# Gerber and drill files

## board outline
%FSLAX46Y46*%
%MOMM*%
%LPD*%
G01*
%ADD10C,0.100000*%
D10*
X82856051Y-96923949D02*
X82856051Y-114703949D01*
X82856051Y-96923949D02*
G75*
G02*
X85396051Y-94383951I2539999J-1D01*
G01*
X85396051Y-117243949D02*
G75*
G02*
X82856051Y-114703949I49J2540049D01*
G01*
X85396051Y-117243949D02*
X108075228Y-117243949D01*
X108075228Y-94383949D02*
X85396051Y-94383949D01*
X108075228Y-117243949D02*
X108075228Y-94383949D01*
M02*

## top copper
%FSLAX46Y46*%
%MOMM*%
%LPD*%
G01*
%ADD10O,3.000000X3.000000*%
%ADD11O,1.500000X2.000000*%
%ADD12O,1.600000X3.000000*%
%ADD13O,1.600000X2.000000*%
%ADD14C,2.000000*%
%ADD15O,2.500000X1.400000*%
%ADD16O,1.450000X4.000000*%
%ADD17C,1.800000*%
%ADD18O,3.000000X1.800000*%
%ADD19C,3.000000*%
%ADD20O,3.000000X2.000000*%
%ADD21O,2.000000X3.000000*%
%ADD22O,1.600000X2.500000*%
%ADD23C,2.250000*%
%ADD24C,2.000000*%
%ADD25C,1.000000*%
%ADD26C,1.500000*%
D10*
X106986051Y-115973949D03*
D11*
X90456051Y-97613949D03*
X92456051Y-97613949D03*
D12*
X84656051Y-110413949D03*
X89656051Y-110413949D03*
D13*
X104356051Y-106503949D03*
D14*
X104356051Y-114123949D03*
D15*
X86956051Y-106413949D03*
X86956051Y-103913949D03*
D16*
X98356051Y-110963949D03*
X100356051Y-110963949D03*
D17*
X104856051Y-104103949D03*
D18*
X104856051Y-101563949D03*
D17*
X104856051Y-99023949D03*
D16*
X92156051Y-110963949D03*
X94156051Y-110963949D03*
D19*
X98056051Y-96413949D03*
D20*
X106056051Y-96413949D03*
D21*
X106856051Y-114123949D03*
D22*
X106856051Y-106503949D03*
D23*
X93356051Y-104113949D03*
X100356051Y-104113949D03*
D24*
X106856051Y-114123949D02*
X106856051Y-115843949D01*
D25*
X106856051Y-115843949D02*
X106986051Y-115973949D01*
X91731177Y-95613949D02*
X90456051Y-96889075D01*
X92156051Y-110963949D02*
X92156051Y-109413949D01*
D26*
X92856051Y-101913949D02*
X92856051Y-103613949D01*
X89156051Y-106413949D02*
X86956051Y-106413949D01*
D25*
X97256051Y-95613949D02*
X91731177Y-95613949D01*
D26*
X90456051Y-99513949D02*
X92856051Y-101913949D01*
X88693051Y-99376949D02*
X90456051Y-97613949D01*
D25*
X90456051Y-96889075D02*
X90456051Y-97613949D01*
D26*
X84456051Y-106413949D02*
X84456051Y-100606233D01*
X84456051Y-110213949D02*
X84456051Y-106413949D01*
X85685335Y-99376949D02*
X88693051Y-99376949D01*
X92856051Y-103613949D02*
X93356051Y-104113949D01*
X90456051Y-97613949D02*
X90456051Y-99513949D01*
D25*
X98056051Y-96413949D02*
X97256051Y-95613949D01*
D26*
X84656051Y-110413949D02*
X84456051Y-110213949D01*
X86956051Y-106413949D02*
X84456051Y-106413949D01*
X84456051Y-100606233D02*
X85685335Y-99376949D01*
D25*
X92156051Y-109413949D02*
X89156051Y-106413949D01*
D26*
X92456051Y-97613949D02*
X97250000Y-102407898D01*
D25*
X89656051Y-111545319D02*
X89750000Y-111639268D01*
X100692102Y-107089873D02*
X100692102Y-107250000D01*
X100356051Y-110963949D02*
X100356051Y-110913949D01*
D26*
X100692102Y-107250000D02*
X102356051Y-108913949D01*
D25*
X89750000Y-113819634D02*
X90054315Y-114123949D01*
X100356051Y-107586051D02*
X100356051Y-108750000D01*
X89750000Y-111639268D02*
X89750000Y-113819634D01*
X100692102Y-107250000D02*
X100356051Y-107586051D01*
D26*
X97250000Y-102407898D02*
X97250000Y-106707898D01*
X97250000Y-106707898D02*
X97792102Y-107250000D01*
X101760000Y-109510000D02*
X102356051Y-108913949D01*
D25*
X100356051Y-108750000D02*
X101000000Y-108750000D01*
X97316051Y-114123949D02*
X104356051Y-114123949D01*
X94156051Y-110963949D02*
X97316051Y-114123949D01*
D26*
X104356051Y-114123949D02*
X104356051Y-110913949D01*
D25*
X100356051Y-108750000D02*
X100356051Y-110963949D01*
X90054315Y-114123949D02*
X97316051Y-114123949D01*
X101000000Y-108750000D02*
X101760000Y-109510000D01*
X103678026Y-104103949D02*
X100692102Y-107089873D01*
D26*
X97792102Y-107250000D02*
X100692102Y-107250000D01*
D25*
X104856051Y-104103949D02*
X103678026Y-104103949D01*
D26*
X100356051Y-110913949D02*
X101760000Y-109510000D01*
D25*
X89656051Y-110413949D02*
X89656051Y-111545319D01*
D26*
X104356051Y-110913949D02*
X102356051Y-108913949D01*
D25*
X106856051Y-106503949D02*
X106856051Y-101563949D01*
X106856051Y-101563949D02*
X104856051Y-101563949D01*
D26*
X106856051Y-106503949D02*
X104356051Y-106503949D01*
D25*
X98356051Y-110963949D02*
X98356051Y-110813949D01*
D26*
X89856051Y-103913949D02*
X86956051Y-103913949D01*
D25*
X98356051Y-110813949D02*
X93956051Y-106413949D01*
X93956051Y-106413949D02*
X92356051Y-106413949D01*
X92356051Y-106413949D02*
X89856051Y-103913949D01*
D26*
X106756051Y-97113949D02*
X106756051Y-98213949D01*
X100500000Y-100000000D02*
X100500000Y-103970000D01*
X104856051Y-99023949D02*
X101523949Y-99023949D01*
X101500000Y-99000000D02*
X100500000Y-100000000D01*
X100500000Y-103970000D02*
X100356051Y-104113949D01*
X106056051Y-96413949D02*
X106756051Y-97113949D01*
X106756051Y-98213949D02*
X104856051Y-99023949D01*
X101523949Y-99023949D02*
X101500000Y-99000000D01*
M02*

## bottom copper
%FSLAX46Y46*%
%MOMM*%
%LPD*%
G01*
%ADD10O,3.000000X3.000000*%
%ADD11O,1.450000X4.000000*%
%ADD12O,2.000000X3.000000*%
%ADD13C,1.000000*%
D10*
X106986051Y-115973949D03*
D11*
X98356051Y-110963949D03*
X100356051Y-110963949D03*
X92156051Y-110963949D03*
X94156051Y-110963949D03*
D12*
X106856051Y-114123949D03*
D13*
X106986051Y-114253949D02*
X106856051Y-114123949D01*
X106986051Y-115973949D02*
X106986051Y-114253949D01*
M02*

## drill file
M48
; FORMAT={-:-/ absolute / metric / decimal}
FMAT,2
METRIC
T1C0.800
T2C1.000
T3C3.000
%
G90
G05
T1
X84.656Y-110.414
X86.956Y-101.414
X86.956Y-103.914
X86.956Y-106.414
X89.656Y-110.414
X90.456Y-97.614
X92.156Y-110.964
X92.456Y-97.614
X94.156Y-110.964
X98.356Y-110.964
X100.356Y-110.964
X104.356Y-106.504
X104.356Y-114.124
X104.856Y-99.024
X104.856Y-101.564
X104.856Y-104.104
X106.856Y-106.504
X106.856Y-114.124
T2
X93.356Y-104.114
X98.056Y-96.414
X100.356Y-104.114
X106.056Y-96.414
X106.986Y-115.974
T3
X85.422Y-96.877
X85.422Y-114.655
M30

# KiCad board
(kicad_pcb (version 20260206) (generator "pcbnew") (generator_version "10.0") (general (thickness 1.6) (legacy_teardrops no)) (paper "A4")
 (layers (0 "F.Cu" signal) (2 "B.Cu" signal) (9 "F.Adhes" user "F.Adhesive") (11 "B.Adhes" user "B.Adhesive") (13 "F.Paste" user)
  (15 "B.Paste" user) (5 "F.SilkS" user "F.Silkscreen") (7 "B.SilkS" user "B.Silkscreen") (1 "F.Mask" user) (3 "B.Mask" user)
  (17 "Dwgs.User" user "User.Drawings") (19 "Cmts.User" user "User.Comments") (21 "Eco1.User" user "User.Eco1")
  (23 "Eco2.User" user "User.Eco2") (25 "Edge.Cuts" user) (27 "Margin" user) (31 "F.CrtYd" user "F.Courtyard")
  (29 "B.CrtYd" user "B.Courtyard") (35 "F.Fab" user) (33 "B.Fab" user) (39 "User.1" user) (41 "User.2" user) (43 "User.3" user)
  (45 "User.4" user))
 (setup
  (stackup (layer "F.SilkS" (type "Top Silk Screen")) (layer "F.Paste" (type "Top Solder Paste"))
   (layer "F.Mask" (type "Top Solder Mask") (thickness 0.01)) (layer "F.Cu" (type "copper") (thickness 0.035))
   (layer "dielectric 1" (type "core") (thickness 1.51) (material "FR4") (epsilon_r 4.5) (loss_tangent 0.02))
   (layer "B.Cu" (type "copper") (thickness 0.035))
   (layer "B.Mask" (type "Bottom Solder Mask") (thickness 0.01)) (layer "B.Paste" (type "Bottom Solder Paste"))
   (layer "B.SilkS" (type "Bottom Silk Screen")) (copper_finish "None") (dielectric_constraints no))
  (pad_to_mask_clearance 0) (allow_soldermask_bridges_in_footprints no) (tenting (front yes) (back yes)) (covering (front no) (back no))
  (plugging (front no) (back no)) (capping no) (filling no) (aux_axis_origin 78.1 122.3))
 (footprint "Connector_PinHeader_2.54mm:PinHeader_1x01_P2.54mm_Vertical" (layer "F.Cu") (at 106.986051 115.973949 180)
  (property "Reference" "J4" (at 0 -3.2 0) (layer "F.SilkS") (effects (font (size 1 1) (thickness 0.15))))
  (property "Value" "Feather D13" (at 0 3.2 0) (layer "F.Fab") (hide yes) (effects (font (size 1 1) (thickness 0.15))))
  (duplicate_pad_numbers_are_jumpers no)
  (pad "e" thru_hole oval (at 0 0 180) (size 3 3) (drill 1) (layers "*.Cu" "F.Mask") (remove_unused_layers no) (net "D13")))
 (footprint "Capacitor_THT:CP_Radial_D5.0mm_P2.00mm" (layer "F.Cu") (at 91.456051 97.613949)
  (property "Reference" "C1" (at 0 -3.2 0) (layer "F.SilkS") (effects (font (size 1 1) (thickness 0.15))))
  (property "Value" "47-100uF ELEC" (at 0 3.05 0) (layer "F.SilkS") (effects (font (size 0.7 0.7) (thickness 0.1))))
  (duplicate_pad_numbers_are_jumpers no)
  (pad "1" thru_hole oval (at -1 0) (size 1.5 2) (drill 0.8) (layers "*.Cu" "F.Mask") (remove_unused_layers yes) (keep_end_layers no)
   (zone_layer_connections) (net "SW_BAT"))
  (pad "2" thru_hole oval (at 1 0) (size 1.5 2) (drill 0.8) (layers "*.Cu" "F.Mask") (remove_unused_layers yes) (keep_end_layers no)
   (zone_layer_connections) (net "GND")))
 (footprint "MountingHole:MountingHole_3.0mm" (layer "F.Cu") (at 85.422051 96.876949 180)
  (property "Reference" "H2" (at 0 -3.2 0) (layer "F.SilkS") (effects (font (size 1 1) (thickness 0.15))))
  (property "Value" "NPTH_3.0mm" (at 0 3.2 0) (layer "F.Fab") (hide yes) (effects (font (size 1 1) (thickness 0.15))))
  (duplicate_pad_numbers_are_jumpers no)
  (pad "" np_thru_hole circle (at 0 0 180) (size 3 3) (drill 3) (layers "*.Cu" "*.Mask")))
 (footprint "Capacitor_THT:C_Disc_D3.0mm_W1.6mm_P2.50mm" (layer "F.Cu") (at 87.156051 110.413949)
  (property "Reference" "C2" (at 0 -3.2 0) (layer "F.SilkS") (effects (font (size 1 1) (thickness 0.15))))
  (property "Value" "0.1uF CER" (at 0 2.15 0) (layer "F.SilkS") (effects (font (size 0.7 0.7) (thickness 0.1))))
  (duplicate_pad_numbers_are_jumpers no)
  (pad "1" thru_hole oval (at -2.5 0) (size 1.6 3) (drill 0.8) (layers "*.Cu" "F.Mask") (remove_unused_layers yes) (keep_end_layers no)
   (zone_layer_connections) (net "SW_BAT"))
  (pad "2" thru_hole oval (at 2.5 0) (size 1.6 3) (drill 0.8) (layers "*.Cu" "F.Mask") (remove_unused_layers yes) (keep_end_layers no)
   (zone_layer_connections) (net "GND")))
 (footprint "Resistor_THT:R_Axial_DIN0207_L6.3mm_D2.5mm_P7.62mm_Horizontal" (layer "F.Cu") (at 104.356051 110.313949 -90)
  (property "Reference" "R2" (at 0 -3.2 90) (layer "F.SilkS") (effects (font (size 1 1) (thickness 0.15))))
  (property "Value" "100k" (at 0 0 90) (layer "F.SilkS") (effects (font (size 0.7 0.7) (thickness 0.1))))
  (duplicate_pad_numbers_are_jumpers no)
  (pad "1" thru_hole oval (at -3.81 0 270) (size 2 1.6) (drill 0.8) (layers "*.Cu" "F.Mask") (remove_unused_layers yes) (keep_end_layers no)
   (zone_layer_connections) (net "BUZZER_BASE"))
  (pad "2" thru_hole circle (at 3.81 0 270) (size 2 2) (drill 0.8) (layers "*.Cu" "F.Mask") (remove_unused_layers yes) (keep_end_layers no)
   (zone_layer_connections) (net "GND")))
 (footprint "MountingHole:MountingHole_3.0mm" (layer "F.Cu") (at 85.422051 114.655349 180)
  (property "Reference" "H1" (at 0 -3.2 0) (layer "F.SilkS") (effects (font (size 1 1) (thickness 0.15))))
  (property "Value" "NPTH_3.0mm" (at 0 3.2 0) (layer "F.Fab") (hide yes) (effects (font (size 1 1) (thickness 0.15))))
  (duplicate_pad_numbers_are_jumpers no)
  (pad "" np_thru_hole circle (at 0 0 180) (size 3 3) (drill 3) (layers "*.Cu" "*.Mask")))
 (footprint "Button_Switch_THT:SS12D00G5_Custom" (layer "F.Cu") (at 86.956051 103.913949 90)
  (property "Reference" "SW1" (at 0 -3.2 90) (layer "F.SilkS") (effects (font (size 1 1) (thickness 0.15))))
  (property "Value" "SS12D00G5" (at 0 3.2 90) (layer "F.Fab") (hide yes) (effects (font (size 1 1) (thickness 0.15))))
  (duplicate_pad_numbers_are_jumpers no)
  (pad "1" thru_hole oval (at -2.5 0 90) (size 1.4 2.5) (drill 0.8) (layers "*.Cu" "F.Mask") (remove_unused_layers yes) (keep_end_layers no)
   (zone_layer_connections) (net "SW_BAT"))
  (pad "2" thru_hole oval (at 0 0 90) (size 1.4 2.5) (drill 0.8) (layers "*.Cu" "F.Mask") (remove_unused_layers yes) (keep_end_layers no)
   (zone_layer_connections) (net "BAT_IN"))
  (pad "3" thru_hole oval (at 2.5 0 90) (size 1.4 2.5) (drill 0.8) (layers "*.Cu" "F.Mask") (remove_unused_layers yes) (keep_end_layers no)
   (zone_layer_connections)))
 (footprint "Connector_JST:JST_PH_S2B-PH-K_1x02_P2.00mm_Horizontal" (layer "F.Cu") (at 99.356051 112.713949)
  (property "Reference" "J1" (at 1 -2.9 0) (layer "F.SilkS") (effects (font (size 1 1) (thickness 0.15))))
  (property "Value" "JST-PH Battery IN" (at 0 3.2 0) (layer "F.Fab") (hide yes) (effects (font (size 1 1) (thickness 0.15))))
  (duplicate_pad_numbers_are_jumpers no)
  (pad "1" thru_hole oval (at -1 -1.75) (size 1.45 4) (drill 0.8) (layers "*.Cu" "F.Mask") (remove_unused_layers no) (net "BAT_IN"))
  (pad "2" thru_hole oval (at 1 -1.75) (size 1.45 4) (drill 0.8) (layers "*.Cu" "F.Mask") (remove_unused_layers no) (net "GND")))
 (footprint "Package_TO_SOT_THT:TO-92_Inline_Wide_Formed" (layer "F.Cu") (at 104.856051 101.563949 90)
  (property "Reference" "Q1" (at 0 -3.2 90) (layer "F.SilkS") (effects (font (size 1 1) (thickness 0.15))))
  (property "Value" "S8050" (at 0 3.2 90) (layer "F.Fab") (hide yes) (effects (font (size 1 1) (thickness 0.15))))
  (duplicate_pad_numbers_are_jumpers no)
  (pad "1" thru_hole circle (at -2.54 0 90) (size 1.8 1.8) (drill 0.8) (layers "*.Cu" "F.Mask") (remove_unused_layers yes)
   (keep_end_layers no) (zone_layer_connections) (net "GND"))
  (pad "2" thru_hole oval (at 0 0 90) (size 1.8 3) (drill 0.8) (layers "*.Cu" "F.Mask") (remove_unused_layers yes) (keep_end_layers no)
   (zone_layer_connections) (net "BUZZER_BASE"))
  (pad "3" thru_hole circle (at 2.54 0 90) (size 1.8 1.8) (drill 0.8) (layers "*.Cu" "F.Mask") (remove_unused_layers yes)
   (keep_end_layers no) (zone_layer_connections) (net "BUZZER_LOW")))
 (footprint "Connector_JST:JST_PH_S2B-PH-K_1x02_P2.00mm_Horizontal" (layer "F.Cu") (at 93.156051 112.713949)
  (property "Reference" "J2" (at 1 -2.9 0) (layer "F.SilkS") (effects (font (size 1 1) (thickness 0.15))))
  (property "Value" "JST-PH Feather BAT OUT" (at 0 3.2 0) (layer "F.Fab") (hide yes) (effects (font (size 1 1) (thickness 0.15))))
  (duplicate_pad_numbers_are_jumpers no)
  (pad "1" thru_hole oval (at -1 -1.75) (size 1.45 4) (drill 0.8) (layers "*.Cu" "F.Mask") (remove_unused_layers no) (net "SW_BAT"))
  (pad "2" thru_hole oval (at 1 -1.75) (size 1.45 4) (drill 0.8) (layers "*.Cu" "F.Mask") (remove_unused_layers no) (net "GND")))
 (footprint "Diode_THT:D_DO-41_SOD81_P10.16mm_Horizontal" (layer "F.Cu") (at 102.056051 96.413949)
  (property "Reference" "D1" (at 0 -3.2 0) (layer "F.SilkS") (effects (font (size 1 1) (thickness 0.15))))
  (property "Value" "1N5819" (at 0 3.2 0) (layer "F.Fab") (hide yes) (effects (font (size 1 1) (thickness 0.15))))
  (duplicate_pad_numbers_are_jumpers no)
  (pad "1" thru_hole circle (at -4 0) (size 3 3) (drill 1) (layers "*.Cu" "F.Mask") (remove_unused_layers yes) (keep_end_layers no)
   (zone_layer_connections) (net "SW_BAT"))
  (pad "2" thru_hole oval (at 4 0) (size 3 2) (drill 1) (layers "*.Cu" "F.Mask") (remove_unused_layers yes) (keep_end_layers no)
   (zone_layer_connections) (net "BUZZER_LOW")))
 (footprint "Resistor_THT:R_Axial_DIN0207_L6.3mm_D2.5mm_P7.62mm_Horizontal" (layer "F.Cu") (at 106.856051 110.313949 90)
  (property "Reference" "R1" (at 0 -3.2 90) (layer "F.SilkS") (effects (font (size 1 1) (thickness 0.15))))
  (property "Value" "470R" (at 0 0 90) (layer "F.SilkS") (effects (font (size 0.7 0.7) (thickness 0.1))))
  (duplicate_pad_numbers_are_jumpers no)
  (pad "1" thru_hole oval (at -3.81 0 90) (size 3 2) (drill 0.8) (layers "*.Cu" "F.Mask") (remove_unused_layers no) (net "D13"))
  (pad "2" thru_hole oval (at 3.81 0 90) (size 2.5 1.6) (drill 0.8) (layers "*.Cu" "F.Mask") (remove_unused_layers yes) (keep_end_layers no)
   (zone_layer_connections) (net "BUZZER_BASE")))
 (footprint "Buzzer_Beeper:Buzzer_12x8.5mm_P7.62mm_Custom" (layer "F.Cu") (at 96.856051 104.113949)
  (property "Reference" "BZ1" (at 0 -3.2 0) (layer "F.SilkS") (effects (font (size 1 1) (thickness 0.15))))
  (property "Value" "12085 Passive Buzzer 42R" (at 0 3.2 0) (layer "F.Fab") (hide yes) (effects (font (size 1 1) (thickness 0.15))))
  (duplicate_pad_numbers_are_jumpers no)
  (pad "1" thru_hole circle (at -3.5 0) (size 2.25 2.25) (drill 1) (layers "*.Cu" "F.Mask") (remove_unused_layers yes) (keep_end_layers no)
   (zone_layer_connections) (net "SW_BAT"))
  (pad "2" thru_hole circle (at 3.5 0) (size 2.25 2.25) (drill 1) (layers "*.Cu" "F.Mask") (remove_unused_layers yes) (keep_end_layers no)
   (zone_layer_connections) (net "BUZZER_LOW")))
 (gr_line (start 82.856051 96.923949) (end 82.856051 114.703949) (stroke (width 0.1) (type default)) (layer "Edge.Cuts"))
 (gr_arc (start 82.856051 96.923949) (mid 83.6 95.127898) (end 85.396051 94.383949) (stroke (width 0.1) (type default)) (layer "Edge.Cuts"))
 (gr_arc (start 85.396051 117.243949) (mid 83.6 116.5) (end 82.856051 114.703949) (stroke (width 0.1) (type default)) (layer "Edge.Cuts"))
 (gr_line (start 85.396051 117.243949) (end 108.075228 117.243949) (stroke (width 0.1) (type default)) (layer "Edge.Cuts"))
 (gr_line (start 108.075228 94.383949) (end 85.396051 94.383949) (stroke (width 0.1) (type default)) (layer "Edge.Cuts"))
 (gr_line (start 108.075228 117.243949) (end 108.075228 94.383949) (stroke (width 0.1) (type default)) (layer "Edge.Cuts"))
 (segment (start 106.856051 114.123949) (end 106.856051 115.843949) (width 2) (layer "F.Cu") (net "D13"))
 (segment (start 106.856051 115.843949) (end 106.986051 115.973949) (width 1) (layer "F.Cu") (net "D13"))
 (segment (start 106.986051 114.253949) (end 106.856051 114.123949) (width 1) (layer "B.Cu") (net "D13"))
 (segment (start 106.986051 115.973949) (end 106.986051 114.253949) (width 1) (layer "B.Cu") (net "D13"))
 (segment (start 91.731177 95.613949) (end 90.456051 96.889075) (width 1) (layer "F.Cu") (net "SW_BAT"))
 (segment (start 92.156051 110.963949) (end 92.156051 109.413949) (width 1) (layer "F.Cu") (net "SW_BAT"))
 (segment (start 92.856051 101.913949) (end 92.856051 103.613949) (width 1.5) (layer "F.Cu") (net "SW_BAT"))
 (segment (start 89.156051 106.413949) (end 86.956051 106.413949) (width 1.5) (layer "F.Cu") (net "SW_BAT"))
 (segment (start 97.256051 95.613949) (end 91.731177 95.613949) (width 1) (layer "F.Cu") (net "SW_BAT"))
 (segment (start 90.456051 99.513949) (end 92.856051 101.913949) (width 1.5) (layer "F.Cu") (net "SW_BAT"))
 (segment (start 88.693051 99.376949) (end 90.456051 97.613949) (width 1.5) (layer "F.Cu") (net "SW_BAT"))
 (segment (start 90.456051 96.889075) (end 90.456051 97.613949) (width 1) (layer "F.Cu") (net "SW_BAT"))
 (segment (start 84.456051 106.413949) (end 84.456051 100.606233) (width 1.5) (layer "F.Cu") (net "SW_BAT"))
 (segment (start 84.456051 110.213949) (end 84.456051 106.413949) (width 1.5) (layer "F.Cu") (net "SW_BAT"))
 (segment (start 85.685335 99.376949) (end 88.693051 99.376949) (width 1.5) (layer "F.Cu") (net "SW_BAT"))
 (segment (start 92.856051 103.613949) (end 93.356051 104.113949) (width 1.5) (layer "F.Cu") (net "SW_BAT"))
 (segment (start 90.456051 97.613949) (end 90.456051 99.513949) (width 1.5) (layer "F.Cu") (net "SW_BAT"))
 (segment (start 98.056051 96.413949) (end 97.256051 95.613949) (width 1) (layer "F.Cu") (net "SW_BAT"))
 (segment (start 84.656051 110.413949) (end 84.456051 110.213949) (width 1.5) (layer "F.Cu") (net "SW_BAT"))
 (segment (start 86.956051 106.413949) (end 84.456051 106.413949) (width 1.5) (layer "F.Cu") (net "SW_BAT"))
 (segment (start 84.456051 100.606233) (end 85.685335 99.376949) (width 1.5) (layer "F.Cu") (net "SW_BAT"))
 (segment (start 92.156051 109.413949) (end 89.156051 106.413949) (width 1) (layer "F.Cu") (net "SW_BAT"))
 (segment (start 92.456051 97.613949) (end 97.25 102.407898) (width 1.5) (layer "F.Cu") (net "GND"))
 (segment (start 89.656051 111.545319) (end 89.75 111.639268) (width 1) (layer "F.Cu") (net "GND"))
 (segment (start 100.692102 107.089873) (end 100.692102 107.25) (width 1) (layer "F.Cu") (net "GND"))
 (segment (start 100.356051 110.963949) (end 100.356051 110.913949) (width 1) (layer "F.Cu") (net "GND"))
 (segment (start 100.692102 107.25) (end 102.356051 108.913949) (width 1.5) (layer "F.Cu") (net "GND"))
 (segment (start 89.75 113.819634) (end 90.054315 114.123949) (width 1) (layer "F.Cu") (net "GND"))
 (segment (start 100.356051 107.586051) (end 100.356051 108.75) (width 1) (layer "F.Cu") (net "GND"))
 (segment (start 89.75 111.639268) (end 89.75 113.819634) (width 1) (layer "F.Cu") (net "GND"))
 (segment (start 100.692102 107.25) (end 100.356051 107.586051) (width 1) (layer "F.Cu") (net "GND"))
 (segment (start 97.25 102.407898) (end 97.25 106.707898) (width 1.5) (layer "F.Cu") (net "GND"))
 (segment (start 97.25 106.707898) (end 97.792102 107.25) (width 1.5) (layer "F.Cu") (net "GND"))
 (segment (start 101.76 109.51) (end 102.356051 108.913949) (width 1.5) (layer "F.Cu") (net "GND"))
 (segment (start 100.356051 108.75) (end 101 108.75) (width 1) (layer "F.Cu") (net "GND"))
 (segment (start 97.316051 114.123949) (end 104.356051 114.123949) (width 1) (layer "F.Cu") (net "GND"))
 (segment (start 94.156051 110.963949) (end 97.316051 114.123949) (width 1) (layer "F.Cu") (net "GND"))
 (segment (start 104.356051 114.123949) (end 104.356051 110.913949) (width 1.5) (layer "F.Cu") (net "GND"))
 (segment (start 100.356051 108.75) (end 100.356051 110.963949) (width 1) (layer "F.Cu") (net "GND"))
 (segment (start 90.054315 114.123949) (end 97.316051 114.123949) (width 1) (layer "F.Cu") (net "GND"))
 (segment (start 101 108.75) (end 101.76 109.51) (width 1) (layer "F.Cu") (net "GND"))
 (segment (start 103.678026 104.103949) (end 100.692102 107.089873) (width 1) (layer "F.Cu") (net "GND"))
 (segment (start 97.792102 107.25) (end 100.692102 107.25) (width 1.5) (layer "F.Cu") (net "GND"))
 (segment (start 104.856051 104.103949) (end 103.678026 104.103949) (width 1) (layer "F.Cu") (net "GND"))
 (segment (start 100.356051 110.913949) (end 101.76 109.51) (width 1.5) (layer "F.Cu") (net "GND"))
 (segment (start 89.656051 110.413949) (end 89.656051 111.545319) (width 1) (layer "F.Cu") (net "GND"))
 (segment (start 104.356051 110.913949) (end 102.356051 108.913949) (width 1.5) (layer "F.Cu") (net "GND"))
 (segment (start 106.856051 106.503949) (end 106.856051 101.563949) (width 1) (layer "F.Cu") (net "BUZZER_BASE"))
 (segment (start 106.856051 101.563949) (end 104.856051 101.563949) (width 1) (layer "F.Cu") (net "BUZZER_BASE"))
 (segment (start 106.856051 106.503949) (end 104.356051 106.503949) (width 1.5) (layer "F.Cu") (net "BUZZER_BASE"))
 (segment (start 98.356051 110.963949) (end 98.356051 110.813949) (width 1) (layer "F.Cu") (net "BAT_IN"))
 (segment (start 89.856051 103.913949) (end 86.956051 103.913949) (width 1.5) (layer "F.Cu") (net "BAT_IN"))
 (segment (start 98.356051 110.813949) (end 93.956051 106.413949) (width 1) (layer "F.Cu") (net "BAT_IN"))
 (segment (start 93.956051 106.413949) (end 92.356051 106.413949) (width 1) (layer "F.Cu") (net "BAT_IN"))
 (segment (start 92.356051 106.413949) (end 89.856051 103.913949) (width 1) (layer "F.Cu") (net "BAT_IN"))
 (segment (start 106.756051 97.113949) (end 106.756051 98.213949) (width 1.5) (layer "F.Cu") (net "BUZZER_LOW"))
 (segment (start 100.5 100) (end 100.5 103.97) (width 1.5) (layer "F.Cu") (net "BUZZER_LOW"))
 (segment (start 104.856051 99.023949) (end 101.523949 99.023949) (width 1.5) (layer "F.Cu") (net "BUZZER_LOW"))
 (segment (start 101.5 99) (end 100.5 100) (width 1.5) (layer "F.Cu") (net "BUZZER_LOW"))
 (segment (start 100.5 103.97) (end 100.356051 104.113949) (width 1.5) (layer "F.Cu") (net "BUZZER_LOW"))
 (segment (start 106.056051 96.413949) (end 106.756051 97.113949) (width 1.5) (layer "F.Cu") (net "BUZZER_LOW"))
 (segment (start 106.756051 98.213949) (end 104.856051 99.023949) (width 1.5) (layer "F.Cu") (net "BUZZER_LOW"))
 (segment (start 101.523949 99.023949) (end 101.5 99) (width 1.5) (layer "F.Cu") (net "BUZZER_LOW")))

